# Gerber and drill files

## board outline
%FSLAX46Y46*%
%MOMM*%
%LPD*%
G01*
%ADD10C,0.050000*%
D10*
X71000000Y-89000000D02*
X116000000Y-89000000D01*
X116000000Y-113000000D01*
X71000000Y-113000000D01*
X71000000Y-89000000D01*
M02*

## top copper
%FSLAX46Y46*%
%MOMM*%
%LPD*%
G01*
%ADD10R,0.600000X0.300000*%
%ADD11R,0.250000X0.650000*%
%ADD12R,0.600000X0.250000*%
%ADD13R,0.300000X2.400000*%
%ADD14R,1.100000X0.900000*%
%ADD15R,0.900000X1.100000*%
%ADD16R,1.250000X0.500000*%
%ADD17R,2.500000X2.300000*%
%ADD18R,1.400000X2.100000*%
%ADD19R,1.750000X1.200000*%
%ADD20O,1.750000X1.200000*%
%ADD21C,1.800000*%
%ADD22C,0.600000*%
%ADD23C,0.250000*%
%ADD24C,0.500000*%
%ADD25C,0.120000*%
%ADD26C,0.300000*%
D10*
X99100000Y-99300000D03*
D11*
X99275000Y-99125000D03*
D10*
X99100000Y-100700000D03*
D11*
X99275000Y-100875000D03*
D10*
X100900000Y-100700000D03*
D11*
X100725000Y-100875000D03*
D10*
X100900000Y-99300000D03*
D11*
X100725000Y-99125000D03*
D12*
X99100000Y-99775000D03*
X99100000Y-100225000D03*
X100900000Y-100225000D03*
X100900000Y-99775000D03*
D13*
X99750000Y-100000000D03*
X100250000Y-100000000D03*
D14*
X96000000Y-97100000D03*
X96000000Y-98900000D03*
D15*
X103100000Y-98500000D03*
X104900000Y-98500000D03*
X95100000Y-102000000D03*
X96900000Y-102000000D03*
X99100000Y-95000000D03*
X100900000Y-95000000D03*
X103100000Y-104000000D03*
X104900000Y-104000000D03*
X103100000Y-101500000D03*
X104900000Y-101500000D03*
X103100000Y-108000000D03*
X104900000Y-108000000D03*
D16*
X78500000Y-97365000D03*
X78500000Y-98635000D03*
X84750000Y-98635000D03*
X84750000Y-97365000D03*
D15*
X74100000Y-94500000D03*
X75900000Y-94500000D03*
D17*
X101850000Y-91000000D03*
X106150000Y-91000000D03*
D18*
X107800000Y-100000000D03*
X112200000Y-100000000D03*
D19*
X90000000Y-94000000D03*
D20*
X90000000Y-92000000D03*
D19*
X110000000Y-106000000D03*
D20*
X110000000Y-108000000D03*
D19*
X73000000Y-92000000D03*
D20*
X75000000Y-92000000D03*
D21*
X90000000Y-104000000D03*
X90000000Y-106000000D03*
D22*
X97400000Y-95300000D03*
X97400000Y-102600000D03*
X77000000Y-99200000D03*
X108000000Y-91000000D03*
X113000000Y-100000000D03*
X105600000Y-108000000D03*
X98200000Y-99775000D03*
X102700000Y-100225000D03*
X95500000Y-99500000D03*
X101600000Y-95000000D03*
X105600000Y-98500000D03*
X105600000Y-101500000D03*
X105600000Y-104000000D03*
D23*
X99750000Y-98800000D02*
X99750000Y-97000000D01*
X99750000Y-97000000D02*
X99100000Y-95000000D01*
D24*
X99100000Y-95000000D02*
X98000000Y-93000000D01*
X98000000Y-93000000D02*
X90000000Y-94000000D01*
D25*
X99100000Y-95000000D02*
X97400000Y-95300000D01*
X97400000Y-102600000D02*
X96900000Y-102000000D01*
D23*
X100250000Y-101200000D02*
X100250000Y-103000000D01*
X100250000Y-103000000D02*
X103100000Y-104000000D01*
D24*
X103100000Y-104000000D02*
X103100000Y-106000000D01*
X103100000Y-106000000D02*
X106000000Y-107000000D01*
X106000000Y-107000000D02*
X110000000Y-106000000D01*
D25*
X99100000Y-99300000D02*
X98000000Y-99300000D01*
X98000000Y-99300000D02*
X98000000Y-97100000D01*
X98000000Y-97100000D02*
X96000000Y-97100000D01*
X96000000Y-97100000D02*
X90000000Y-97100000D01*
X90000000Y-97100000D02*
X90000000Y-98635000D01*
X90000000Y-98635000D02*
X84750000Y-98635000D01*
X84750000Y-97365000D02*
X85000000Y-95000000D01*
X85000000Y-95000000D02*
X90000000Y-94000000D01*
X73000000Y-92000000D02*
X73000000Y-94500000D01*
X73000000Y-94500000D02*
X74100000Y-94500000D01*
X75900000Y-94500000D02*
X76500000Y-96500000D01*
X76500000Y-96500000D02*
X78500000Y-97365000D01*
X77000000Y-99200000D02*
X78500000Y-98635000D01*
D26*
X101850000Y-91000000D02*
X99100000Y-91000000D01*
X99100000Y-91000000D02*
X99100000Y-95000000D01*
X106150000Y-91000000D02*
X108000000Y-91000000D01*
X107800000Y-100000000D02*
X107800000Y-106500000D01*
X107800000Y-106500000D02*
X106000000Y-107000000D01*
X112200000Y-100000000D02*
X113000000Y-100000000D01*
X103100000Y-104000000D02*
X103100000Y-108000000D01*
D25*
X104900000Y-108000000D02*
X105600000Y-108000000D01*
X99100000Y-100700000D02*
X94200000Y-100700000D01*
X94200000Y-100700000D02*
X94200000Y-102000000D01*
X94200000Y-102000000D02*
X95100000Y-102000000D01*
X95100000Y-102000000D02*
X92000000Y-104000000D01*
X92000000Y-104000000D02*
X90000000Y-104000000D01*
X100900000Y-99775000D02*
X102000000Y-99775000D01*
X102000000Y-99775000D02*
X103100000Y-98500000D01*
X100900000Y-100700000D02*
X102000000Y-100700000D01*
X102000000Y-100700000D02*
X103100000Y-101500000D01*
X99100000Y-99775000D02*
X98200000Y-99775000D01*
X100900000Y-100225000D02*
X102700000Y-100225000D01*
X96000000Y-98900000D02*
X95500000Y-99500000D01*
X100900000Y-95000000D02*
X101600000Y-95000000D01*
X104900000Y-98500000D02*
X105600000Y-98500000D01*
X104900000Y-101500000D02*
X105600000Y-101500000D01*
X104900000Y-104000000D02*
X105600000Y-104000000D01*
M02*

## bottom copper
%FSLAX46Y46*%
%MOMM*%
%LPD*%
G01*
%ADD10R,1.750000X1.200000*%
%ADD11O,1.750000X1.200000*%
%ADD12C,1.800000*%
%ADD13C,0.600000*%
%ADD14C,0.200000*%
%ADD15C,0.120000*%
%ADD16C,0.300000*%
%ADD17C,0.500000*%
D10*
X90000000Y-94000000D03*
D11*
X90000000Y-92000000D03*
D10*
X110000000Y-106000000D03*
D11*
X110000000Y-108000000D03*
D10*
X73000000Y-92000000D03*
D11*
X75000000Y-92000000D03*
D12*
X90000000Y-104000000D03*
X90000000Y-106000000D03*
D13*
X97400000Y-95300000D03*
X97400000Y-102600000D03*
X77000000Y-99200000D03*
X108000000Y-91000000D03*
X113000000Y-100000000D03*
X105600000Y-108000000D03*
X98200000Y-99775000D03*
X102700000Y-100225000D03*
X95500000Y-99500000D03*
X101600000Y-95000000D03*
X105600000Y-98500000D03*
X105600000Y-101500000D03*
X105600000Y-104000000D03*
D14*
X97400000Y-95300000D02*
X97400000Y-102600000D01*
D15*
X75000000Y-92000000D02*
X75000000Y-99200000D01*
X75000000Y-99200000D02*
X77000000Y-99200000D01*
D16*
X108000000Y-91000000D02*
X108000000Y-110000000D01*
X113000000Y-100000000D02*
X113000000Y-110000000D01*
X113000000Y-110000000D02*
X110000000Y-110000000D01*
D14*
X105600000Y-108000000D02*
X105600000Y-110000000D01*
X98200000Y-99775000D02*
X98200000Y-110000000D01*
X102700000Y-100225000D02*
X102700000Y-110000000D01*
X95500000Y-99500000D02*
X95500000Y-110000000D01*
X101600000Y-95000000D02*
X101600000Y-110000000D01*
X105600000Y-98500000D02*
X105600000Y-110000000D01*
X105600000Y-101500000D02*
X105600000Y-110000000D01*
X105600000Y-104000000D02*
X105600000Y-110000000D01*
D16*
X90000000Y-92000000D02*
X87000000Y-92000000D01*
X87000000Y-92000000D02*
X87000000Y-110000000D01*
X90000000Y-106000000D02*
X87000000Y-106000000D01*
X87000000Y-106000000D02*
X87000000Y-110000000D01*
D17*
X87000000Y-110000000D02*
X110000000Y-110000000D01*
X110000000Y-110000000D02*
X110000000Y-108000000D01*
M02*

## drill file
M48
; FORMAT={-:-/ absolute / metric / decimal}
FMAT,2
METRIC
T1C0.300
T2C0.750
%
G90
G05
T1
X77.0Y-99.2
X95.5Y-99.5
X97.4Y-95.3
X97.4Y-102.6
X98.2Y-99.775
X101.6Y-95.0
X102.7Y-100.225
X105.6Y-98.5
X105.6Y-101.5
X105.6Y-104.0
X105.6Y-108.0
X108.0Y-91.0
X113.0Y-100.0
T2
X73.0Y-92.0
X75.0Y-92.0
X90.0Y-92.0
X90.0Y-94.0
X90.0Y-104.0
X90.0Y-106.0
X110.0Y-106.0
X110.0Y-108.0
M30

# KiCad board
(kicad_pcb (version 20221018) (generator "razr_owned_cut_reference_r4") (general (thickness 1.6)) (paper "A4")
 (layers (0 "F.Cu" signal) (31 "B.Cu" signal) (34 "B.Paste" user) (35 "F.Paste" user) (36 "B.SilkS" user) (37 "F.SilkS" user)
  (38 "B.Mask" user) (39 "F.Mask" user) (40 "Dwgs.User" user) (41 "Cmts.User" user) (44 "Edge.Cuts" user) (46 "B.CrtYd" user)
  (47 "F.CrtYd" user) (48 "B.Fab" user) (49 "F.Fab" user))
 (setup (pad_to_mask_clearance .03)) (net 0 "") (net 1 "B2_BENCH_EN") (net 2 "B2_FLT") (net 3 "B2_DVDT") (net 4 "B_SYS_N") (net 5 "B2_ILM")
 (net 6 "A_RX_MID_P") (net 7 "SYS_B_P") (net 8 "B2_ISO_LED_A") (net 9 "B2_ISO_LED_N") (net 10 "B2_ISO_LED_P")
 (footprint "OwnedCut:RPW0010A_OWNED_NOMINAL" (layer "F.Cu") (at 100 100)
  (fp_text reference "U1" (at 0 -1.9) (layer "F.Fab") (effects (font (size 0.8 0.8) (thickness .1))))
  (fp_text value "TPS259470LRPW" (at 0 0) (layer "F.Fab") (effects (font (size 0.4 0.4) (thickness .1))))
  (pad "1" smd rect (at -0.9 -0.7) (size 0.6 0.3) (layers "F.Cu" "F.Paste" "F.Mask") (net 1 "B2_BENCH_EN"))
  (pad "1" smd rect (at -0.725 -0.875) (size 0.25 0.65) (layers "F.Cu" "F.Paste" "F.Mask") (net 1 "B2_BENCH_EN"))
  (pad "4" smd rect (at -0.9 0.7) (size 0.6 0.3) (layers "F.Cu" "F.Paste" "F.Mask") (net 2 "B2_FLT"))
  (pad "4" smd rect (at -0.725 0.875) (size 0.25 0.65) (layers "F.Cu" "F.Paste" "F.Mask") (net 2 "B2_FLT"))
  (pad "7" smd rect (at 0.9 0.7) (size 0.6 0.3) (layers "F.Cu" "F.Paste" "F.Mask") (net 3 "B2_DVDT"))
  (pad "7" smd rect (at 0.725 0.875) (size 0.25 0.65) (layers "F.Cu" "F.Paste" "F.Mask") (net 3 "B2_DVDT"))
  (pad "10" smd rect (at 0.9 -0.7) (size 0.6 0.3) (layers "F.Cu" "F.Paste" "F.Mask"))
  (pad "10" smd rect (at 0.725 -0.875) (size 0.25 0.65) (layers "F.Cu" "F.Paste" "F.Mask"))
  (pad "2" smd rect (at -0.9 -0.225) (size 0.6 0.25) (layers "F.Cu" "F.Paste" "F.Mask") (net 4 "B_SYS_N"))
  (pad "3" smd rect (at -0.9 0.225) (size 0.6 0.25) (layers "F.Cu" "F.Paste" "F.Mask"))
  (pad "8" smd rect (at 0.9 0.225) (size 0.6 0.25) (layers "F.Cu" "F.Paste" "F.Mask") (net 4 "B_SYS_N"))
  (pad "9" smd rect (at 0.9 -0.225) (size 0.6 0.25) (layers "F.Cu" "F.Paste" "F.Mask") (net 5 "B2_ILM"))
  (pad "5" smd rect (at -0.25 0) (size 0.3 2.4) (layers "F.Cu" "F.Paste" "F.Mask") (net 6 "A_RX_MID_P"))
  (pad "6" smd rect (at 0.25 0) (size 0.3 2.4) (layers "F.Cu" "F.Paste" "F.Mask") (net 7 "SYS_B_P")))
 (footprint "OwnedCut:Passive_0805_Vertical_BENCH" (layer "F.Cu") (at 96 98)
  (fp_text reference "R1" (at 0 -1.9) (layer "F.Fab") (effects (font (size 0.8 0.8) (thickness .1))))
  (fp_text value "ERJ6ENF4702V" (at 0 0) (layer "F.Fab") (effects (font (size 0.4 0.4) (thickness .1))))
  (pad "1" smd rect (at 0 -0.9) (size 1.1 0.9) (layers "F.Cu" "F.Paste" "F.Mask") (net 1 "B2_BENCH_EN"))
  (pad "2" smd rect (at 0 0.9) (size 1.1 0.9) (layers "F.Cu" "F.Paste" "F.Mask") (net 4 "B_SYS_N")))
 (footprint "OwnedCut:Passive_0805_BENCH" (layer "F.Cu") (at 104 98.5)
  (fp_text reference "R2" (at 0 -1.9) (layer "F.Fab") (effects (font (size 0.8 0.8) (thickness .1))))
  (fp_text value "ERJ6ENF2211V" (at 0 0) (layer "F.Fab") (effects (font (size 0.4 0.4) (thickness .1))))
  (pad "1" smd rect (at -0.9 0) (size 0.9 1.1) (layers "F.Cu" "F.Paste" "F.Mask") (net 5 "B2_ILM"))
  (pad "2" smd rect (at 0.9 0) (size 0.9 1.1) (layers "F.Cu" "F.Paste" "F.Mask") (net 4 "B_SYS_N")))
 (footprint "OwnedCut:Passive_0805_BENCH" (layer "F.Cu") (at 96 102)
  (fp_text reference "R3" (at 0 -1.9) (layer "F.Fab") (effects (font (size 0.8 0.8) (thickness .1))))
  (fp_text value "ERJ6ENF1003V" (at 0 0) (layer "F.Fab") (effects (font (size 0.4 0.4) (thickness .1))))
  (pad "1" smd rect (at -0.9 0) (size 0.9 1.1) (layers "F.Cu" "F.Paste" "F.Mask") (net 2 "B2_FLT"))
  (pad "2" smd rect (at 0.9 0) (size 0.9 1.1) (layers "F.Cu" "F.Paste" "F.Mask") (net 6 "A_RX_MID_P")))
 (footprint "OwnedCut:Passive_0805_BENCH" (layer "F.Cu") (at 100 95)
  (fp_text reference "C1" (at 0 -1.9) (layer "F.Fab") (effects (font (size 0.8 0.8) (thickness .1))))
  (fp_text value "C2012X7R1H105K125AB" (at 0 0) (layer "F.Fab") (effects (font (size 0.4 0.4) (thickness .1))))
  (pad "1" smd rect (at -0.9 0) (size 0.9 1.1) (layers "F.Cu" "F.Paste" "F.Mask") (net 6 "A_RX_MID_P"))
  (pad "2" smd rect (at 0.9 0) (size 0.9 1.1) (layers "F.Cu" "F.Paste" "F.Mask") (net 4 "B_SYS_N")))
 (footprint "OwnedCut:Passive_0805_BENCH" (layer "F.Cu") (at 104 104)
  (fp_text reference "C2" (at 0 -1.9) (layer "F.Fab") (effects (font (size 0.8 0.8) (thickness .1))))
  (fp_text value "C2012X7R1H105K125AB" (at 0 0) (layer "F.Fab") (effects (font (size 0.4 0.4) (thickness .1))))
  (pad "1" smd rect (at -0.9 0) (size 0.9 1.1) (layers "F.Cu" "F.Paste" "F.Mask") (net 7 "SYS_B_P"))
  (pad "2" smd rect (at 0.9 0) (size 0.9 1.1) (layers "F.Cu" "F.Paste" "F.Mask") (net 4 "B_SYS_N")))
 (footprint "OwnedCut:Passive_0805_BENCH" (layer "F.Cu") (at 104 101.5)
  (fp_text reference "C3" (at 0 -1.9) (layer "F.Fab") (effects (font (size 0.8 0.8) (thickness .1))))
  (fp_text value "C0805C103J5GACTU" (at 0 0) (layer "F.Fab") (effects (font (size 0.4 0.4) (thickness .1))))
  (pad "1" smd rect (at -0.9 0) (size 0.9 1.1) (layers "F.Cu" "F.Paste" "F.Mask") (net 3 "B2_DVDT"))
  (pad "2" smd rect (at 0.9 0) (size 0.9 1.1) (layers "F.Cu" "F.Paste" "F.Mask") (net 4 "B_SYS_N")))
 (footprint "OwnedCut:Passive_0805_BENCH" (layer "F.Cu") (at 104 108)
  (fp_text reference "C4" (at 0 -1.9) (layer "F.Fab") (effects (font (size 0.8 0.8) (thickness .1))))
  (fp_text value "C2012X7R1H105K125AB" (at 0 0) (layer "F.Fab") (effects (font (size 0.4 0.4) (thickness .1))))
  (pad "1" smd rect (at -0.9 0) (size 0.9 1.1) (layers "F.Cu" "F.Paste" "F.Mask") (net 7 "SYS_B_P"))
  (pad "2" smd rect (at 0.9 0) (size 0.9 1.1) (layers "F.Cu" "F.Paste" "F.Mask") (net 4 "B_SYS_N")))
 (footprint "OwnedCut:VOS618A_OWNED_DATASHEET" (layer "F.Cu") (at 81.625 98)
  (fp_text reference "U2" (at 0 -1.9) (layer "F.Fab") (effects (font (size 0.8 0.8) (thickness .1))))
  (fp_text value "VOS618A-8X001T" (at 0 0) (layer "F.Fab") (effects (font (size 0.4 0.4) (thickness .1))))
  (pad "1" smd rect (at -3.125 -0.635) (size 1.25 0.5) (layers "F.Cu" "F.Paste" "F.Mask") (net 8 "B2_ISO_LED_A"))
  (pad "2" smd rect (at -3.125 0.635) (size 1.25 0.5) (layers "F.Cu" "F.Paste" "F.Mask") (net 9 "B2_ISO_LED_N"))
  (pad "3" smd rect (at 3.125 0.635) (size 1.25 0.5) (layers "F.Cu" "F.Paste" "F.Mask") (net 1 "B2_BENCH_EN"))
  (pad "4" smd rect (at 3.125 -0.635) (size 1.25 0.5) (layers "F.Cu" "F.Paste" "F.Mask") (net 6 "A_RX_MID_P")))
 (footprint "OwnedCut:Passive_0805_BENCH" (layer "F.Cu") (at 75 94.5)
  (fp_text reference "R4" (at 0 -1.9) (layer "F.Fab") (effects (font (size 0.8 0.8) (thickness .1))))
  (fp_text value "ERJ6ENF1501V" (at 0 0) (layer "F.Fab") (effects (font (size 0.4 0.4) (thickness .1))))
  (pad "1" smd rect (at -0.9 0) (size 0.9 1.1) (layers "F.Cu" "F.Paste" "F.Mask") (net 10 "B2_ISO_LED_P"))
  (pad "2" smd rect (at 0.9 0) (size 0.9 1.1) (layers "F.Cu" "F.Paste" "F.Mask") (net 8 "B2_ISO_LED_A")))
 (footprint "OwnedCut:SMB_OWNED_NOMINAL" (layer "F.Cu") (at 104 91)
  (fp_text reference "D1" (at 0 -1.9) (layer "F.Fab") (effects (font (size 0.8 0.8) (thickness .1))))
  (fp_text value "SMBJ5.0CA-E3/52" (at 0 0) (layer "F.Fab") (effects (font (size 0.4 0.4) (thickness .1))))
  (pad "1" smd rect (at -2.15 0) (size 2.5 2.3) (layers "F.Cu" "F.Paste" "F.Mask") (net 6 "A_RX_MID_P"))
  (pad "2" smd rect (at 2.15 0) (size 2.5 2.3) (layers "F.Cu" "F.Paste" "F.Mask") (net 4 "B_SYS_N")))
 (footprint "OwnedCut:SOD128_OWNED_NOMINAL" (layer "F.Cu") (at 110 100)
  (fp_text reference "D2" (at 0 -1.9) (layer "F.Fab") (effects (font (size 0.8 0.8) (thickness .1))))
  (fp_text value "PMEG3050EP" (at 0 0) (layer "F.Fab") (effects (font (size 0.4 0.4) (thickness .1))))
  (pad "1" smd rect (at -2.2 0) (size 1.4 2.1) (layers "F.Cu" "F.Paste" "F.Mask") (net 7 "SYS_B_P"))
  (pad "2" smd rect (at 2.2 0) (size 1.4 2.1) (layers "F.Cu" "F.Paste" "F.Mask") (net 4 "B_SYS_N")))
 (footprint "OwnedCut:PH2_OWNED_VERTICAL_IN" (layer "F.Cu") (at 90 94)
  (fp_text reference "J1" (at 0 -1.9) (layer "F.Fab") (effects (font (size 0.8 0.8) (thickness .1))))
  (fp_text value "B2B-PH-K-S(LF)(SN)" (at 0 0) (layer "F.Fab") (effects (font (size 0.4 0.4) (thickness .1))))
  (pad "1" thru_hole rect (at 0 0) (size 1.75 1.2) (drill .75) (layers "*.Cu" "*.Mask") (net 6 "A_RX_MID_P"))
  (pad "2" thru_hole oval (at 0 -2) (size 1.75 1.2) (drill .75) (layers "*.Cu" "*.Mask") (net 4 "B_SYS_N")))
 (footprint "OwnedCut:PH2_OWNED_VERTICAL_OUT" (layer "F.Cu") (at 110 106)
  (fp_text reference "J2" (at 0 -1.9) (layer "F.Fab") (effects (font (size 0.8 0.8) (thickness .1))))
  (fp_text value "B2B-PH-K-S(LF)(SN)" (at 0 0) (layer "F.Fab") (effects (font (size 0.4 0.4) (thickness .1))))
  (pad "1" thru_hole rect (at 0 0) (size 1.75 1.2) (drill .75) (layers "*.Cu" "*.Mask") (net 7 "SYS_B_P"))
  (pad "2" thru_hole oval (at 0 2) (size 1.75 1.2) (drill .75) (layers "*.Cu" "*.Mask") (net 4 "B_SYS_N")))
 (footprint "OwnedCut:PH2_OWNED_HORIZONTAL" (layer "F.Cu") (at 73 92)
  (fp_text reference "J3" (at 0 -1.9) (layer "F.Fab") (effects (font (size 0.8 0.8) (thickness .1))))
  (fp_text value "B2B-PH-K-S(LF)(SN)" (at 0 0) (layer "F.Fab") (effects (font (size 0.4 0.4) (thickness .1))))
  (pad "1" thru_hole rect (at 0 0) (size 1.75 1.2) (drill .75) (layers "*.Cu" "*.Mask") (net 10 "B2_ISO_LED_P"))
  (pad "2" thru_hole oval (at 2 0) (size 1.75 1.2) (drill .75) (layers "*.Cu" "*.Mask") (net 9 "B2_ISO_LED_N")))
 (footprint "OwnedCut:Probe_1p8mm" (layer "F.Cu") (at 90 104)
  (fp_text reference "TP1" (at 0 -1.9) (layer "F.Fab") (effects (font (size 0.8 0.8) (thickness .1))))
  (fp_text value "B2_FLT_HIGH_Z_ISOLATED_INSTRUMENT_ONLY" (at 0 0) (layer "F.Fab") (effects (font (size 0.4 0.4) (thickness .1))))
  (pad "1" thru_hole circle (at 0 0) (size 1.8 1.8) (drill .75) (layers "*.Cu" "*.Mask") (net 2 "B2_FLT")))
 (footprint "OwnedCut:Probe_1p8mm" (layer "F.Cu") (at 90 106)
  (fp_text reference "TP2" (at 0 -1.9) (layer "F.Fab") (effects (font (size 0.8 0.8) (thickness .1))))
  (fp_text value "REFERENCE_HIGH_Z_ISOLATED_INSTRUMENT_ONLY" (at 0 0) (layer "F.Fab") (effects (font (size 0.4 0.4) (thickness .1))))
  (pad "1" thru_hole circle (at 0 0) (size 1.8 1.8) (drill .75) (layers "*.Cu" "*.Mask") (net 4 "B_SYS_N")))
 (segment (start 99.75 98.8) (end 99.75 97) (width 0.25) (layer "F.Cu") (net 6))
 (segment (start 99.75 97) (end 99.1 95) (width 0.25) (layer "F.Cu") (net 6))
 (segment (start 99.1 95) (end 98 93) (width 0.5) (layer "F.Cu") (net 6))
 (segment (start 98 93) (end 90 94) (width 0.5) (layer "F.Cu") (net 6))
 (segment (start 99.1 95) (end 97.4 95.3) (width 0.12) (layer "F.Cu") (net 6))
 (via (at 97.4 95.3) (size .6) (drill .3) (layers "F.Cu" "B.Cu") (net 6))
 (segment (start 97.4 95.3) (end 97.4 102.6) (width 0.2) (layer "B.Cu") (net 6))
 (via (at 97.4 102.6) (size .6) (drill .3) (layers "F.Cu" "B.Cu") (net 6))
 (segment (start 97.4 102.6) (end 96.9 102) (width 0.12) (layer "F.Cu") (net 6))
 (segment (start 100.25 101.2) (end 100.25 103) (width 0.25) (layer "F.Cu") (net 7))
 (segment (start 100.25 103) (end 103.1 104) (width 0.25) (layer "F.Cu") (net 7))
 (segment (start 103.1 104) (end 103.1 106) (width 0.5) (layer "F.Cu") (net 7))
 (segment (start 103.1 106) (end 106 107) (width 0.5) (layer "F.Cu") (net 7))
 (segment (start 106 107) (end 110 106) (width 0.5) (layer "F.Cu") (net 7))
 (segment (start 99.1 99.3) (end 98 99.3) (width 0.12) (layer "F.Cu") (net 1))
 (segment (start 98 99.3) (end 98 97.1) (width 0.12) (layer "F.Cu") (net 1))
 (segment (start 98 97.1) (end 96 97.1) (width 0.12) (layer "F.Cu") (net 1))
 (segment (start 96 97.1) (end 90 97.1) (width 0.12) (layer "F.Cu") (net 1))
 (segment (start 90 97.1) (end 90 98.635) (width 0.12) (layer "F.Cu") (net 1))
 (segment (start 90 98.635) (end 84.75 98.635) (width 0.12) (layer "F.Cu") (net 1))
 (segment (start 84.75 97.365) (end 85 95) (width 0.12) (layer "F.Cu") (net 6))
 (segment (start 85 95) (end 90 94) (width 0.12) (layer "F.Cu") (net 6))
 (segment (start 73 92) (end 73 94.5) (width 0.12) (layer "F.Cu") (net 10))
 (segment (start 73 94.5) (end 74.1 94.5) (width 0.12) (layer "F.Cu") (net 10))
 (segment (start 75.9 94.5) (end 76.5 96.5) (width 0.12) (layer "F.Cu") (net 8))
 (segment (start 76.5 96.5) (end 78.5 97.365) (width 0.12) (layer "F.Cu") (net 8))
 (segment (start 75 92) (end 75 99.2) (width 0.12) (layer "B.Cu") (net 9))
 (segment (start 75 99.2) (end 77 99.2) (width 0.12) (layer "B.Cu") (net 9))
 (via (at 77 99.2) (size .6) (drill .3) (layers "F.Cu" "B.Cu") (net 9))
 (segment (start 77 99.2) (end 78.5 98.635) (width 0.12) (layer "F.Cu") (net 9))
 (segment (start 101.85 91) (end 99.1 91) (width 0.3) (layer "F.Cu") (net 6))
 (segment (start 99.1 91) (end 99.1 95) (width 0.3) (layer "F.Cu") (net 6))
 (segment (start 106.15 91) (end 108 91) (width 0.3) (layer "F.Cu") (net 4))
 (via (at 108 91) (size .6) (drill .3) (layers "F.Cu" "B.Cu") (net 4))
 (segment (start 108 91) (end 108 110) (width 0.3) (layer "B.Cu") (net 4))
 (segment (start 107.8 100) (end 107.8 106.5) (width 0.3) (layer "F.Cu") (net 7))
 (segment (start 107.8 106.5) (end 106 107) (width 0.3) (layer "F.Cu") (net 7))
 (segment (start 112.2 100) (end 113 100) (width 0.3) (layer "F.Cu") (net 4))
 (via (at 113 100) (size .6) (drill .3) (layers "F.Cu" "B.Cu") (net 4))
 (segment (start 113 100) (end 113 110) (width 0.3) (layer "B.Cu") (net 4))
 (segment (start 113 110) (end 110 110) (width 0.3) (layer "B.Cu") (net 4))
 (segment (start 103.1 104) (end 103.1 108) (width 0.3) (layer "F.Cu") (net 7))
 (segment (start 104.9 108) (end 105.6 108) (width 0.12) (layer "F.Cu") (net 4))
 (via (at 105.6 108) (size .6) (drill .3) (layers "F.Cu" "B.Cu") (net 4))
 (segment (start 105.6 108) (end 105.6 110) (width 0.2) (layer "B.Cu") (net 4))
 (segment (start 99.1 100.7) (end 94.2 100.7) (width 0.12) (layer "F.Cu") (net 2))
 (segment (start 94.2 100.7) (end 94.2 102) (width 0.12) (layer "F.Cu") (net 2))
 (segment (start 94.2 102) (end 95.1 102) (width 0.12) (layer "F.Cu") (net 2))
 (segment (start 95.1 102) (end 92 104) (width 0.12) (layer "F.Cu") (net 2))
 (segment (start 92 104) (end 90 104) (width 0.12) (layer "F.Cu") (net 2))
 (segment (start 100.9 99.775) (end 102 99.775) (width 0.12) (layer "F.Cu") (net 5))
 (segment (start 102 99.775) (end 103.1 98.5) (width 0.12) (layer "F.Cu") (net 5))
 (segment (start 100.9 100.7) (end 102 100.7) (width 0.12) (layer "F.Cu") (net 3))
 (segment (start 102 100.7) (end 103.1 101.5) (width 0.12) (layer "F.Cu") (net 3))
 (segment (start 99.1 99.775) (end 98.2 99.775) (width 0.12) (layer "F.Cu") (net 4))
 (via (at 98.2 99.775) (size .6) (drill .3) (layers "F.Cu" "B.Cu") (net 4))
 (segment (start 98.2 99.775) (end 98.2 110) (width 0.2) (layer "B.Cu") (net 4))
 (segment (start 100.9 100.225) (end 102.7 100.225) (width 0.12) (layer "F.Cu") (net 4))
 (via (at 102.7 100.225) (size .6) (drill .3) (layers "F.Cu" "B.Cu") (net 4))
 (segment (start 102.7 100.225) (end 102.7 110) (width 0.2) (layer "B.Cu") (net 4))
 (segment (start 96 98.9) (end 95.5 99.5) (width 0.12) (layer "F.Cu") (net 4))
 (via (at 95.5 99.5) (size .6) (drill .3) (layers "F.Cu" "B.Cu") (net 4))
 (segment (start 95.5 99.5) (end 95.5 110) (width 0.2) (layer "B.Cu") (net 4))
 (segment (start 100.9 95) (end 101.6 95) (width 0.12) (layer "F.Cu") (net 4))
 (via (at 101.6 95) (size .6) (drill .3) (layers "F.Cu" "B.Cu") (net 4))
 (segment (start 101.6 95) (end 101.6 110) (width 0.2) (layer "B.Cu") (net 4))
 (segment (start 104.9 98.5) (end 105.6 98.5) (width 0.12) (layer "F.Cu") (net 4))
 (via (at 105.6 98.5) (size .6) (drill .3) (layers "F.Cu" "B.Cu") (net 4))
 (segment (start 105.6 98.5) (end 105.6 110) (width 0.2) (layer "B.Cu") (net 4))
 (segment (start 104.9 101.5) (end 105.6 101.5) (width 0.12) (layer "F.Cu") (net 4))
 (via (at 105.6 101.5) (size .6) (drill .3) (layers "F.Cu" "B.Cu") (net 4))
 (segment (start 105.6 101.5) (end 105.6 110) (width 0.2) (layer "B.Cu") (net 4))
 (segment (start 104.9 104) (end 105.6 104) (width 0.12) (layer "F.Cu") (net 4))
 (via (at 105.6 104) (size .6) (drill .3) (layers "F.Cu" "B.Cu") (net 4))
 (segment (start 105.6 104) (end 105.6 110) (width 0.2) (layer "B.Cu") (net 4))
 (segment (start 90 92) (end 87 92) (width 0.3) (layer "B.Cu") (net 4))
 (segment (start 87 92) (end 87 110) (width 0.3) (layer "B.Cu") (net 4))
 (segment (start 90 106) (end 87 106) (width 0.3) (layer "B.Cu") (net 4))
 (segment (start 87 106) (end 87 110) (width 0.3) (layer "B.Cu") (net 4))
 (segment (start 87 110) (end 110 110) (width 0.5) (layer "B.Cu") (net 4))
 (segment (start 110 110) (end 110 108) (width 0.5) (layer "B.Cu") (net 4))
 (gr_rect (start 71 89) (end 116 113) (stroke (width .05) (type default)) (fill none) (layer "Edge.Cuts")))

